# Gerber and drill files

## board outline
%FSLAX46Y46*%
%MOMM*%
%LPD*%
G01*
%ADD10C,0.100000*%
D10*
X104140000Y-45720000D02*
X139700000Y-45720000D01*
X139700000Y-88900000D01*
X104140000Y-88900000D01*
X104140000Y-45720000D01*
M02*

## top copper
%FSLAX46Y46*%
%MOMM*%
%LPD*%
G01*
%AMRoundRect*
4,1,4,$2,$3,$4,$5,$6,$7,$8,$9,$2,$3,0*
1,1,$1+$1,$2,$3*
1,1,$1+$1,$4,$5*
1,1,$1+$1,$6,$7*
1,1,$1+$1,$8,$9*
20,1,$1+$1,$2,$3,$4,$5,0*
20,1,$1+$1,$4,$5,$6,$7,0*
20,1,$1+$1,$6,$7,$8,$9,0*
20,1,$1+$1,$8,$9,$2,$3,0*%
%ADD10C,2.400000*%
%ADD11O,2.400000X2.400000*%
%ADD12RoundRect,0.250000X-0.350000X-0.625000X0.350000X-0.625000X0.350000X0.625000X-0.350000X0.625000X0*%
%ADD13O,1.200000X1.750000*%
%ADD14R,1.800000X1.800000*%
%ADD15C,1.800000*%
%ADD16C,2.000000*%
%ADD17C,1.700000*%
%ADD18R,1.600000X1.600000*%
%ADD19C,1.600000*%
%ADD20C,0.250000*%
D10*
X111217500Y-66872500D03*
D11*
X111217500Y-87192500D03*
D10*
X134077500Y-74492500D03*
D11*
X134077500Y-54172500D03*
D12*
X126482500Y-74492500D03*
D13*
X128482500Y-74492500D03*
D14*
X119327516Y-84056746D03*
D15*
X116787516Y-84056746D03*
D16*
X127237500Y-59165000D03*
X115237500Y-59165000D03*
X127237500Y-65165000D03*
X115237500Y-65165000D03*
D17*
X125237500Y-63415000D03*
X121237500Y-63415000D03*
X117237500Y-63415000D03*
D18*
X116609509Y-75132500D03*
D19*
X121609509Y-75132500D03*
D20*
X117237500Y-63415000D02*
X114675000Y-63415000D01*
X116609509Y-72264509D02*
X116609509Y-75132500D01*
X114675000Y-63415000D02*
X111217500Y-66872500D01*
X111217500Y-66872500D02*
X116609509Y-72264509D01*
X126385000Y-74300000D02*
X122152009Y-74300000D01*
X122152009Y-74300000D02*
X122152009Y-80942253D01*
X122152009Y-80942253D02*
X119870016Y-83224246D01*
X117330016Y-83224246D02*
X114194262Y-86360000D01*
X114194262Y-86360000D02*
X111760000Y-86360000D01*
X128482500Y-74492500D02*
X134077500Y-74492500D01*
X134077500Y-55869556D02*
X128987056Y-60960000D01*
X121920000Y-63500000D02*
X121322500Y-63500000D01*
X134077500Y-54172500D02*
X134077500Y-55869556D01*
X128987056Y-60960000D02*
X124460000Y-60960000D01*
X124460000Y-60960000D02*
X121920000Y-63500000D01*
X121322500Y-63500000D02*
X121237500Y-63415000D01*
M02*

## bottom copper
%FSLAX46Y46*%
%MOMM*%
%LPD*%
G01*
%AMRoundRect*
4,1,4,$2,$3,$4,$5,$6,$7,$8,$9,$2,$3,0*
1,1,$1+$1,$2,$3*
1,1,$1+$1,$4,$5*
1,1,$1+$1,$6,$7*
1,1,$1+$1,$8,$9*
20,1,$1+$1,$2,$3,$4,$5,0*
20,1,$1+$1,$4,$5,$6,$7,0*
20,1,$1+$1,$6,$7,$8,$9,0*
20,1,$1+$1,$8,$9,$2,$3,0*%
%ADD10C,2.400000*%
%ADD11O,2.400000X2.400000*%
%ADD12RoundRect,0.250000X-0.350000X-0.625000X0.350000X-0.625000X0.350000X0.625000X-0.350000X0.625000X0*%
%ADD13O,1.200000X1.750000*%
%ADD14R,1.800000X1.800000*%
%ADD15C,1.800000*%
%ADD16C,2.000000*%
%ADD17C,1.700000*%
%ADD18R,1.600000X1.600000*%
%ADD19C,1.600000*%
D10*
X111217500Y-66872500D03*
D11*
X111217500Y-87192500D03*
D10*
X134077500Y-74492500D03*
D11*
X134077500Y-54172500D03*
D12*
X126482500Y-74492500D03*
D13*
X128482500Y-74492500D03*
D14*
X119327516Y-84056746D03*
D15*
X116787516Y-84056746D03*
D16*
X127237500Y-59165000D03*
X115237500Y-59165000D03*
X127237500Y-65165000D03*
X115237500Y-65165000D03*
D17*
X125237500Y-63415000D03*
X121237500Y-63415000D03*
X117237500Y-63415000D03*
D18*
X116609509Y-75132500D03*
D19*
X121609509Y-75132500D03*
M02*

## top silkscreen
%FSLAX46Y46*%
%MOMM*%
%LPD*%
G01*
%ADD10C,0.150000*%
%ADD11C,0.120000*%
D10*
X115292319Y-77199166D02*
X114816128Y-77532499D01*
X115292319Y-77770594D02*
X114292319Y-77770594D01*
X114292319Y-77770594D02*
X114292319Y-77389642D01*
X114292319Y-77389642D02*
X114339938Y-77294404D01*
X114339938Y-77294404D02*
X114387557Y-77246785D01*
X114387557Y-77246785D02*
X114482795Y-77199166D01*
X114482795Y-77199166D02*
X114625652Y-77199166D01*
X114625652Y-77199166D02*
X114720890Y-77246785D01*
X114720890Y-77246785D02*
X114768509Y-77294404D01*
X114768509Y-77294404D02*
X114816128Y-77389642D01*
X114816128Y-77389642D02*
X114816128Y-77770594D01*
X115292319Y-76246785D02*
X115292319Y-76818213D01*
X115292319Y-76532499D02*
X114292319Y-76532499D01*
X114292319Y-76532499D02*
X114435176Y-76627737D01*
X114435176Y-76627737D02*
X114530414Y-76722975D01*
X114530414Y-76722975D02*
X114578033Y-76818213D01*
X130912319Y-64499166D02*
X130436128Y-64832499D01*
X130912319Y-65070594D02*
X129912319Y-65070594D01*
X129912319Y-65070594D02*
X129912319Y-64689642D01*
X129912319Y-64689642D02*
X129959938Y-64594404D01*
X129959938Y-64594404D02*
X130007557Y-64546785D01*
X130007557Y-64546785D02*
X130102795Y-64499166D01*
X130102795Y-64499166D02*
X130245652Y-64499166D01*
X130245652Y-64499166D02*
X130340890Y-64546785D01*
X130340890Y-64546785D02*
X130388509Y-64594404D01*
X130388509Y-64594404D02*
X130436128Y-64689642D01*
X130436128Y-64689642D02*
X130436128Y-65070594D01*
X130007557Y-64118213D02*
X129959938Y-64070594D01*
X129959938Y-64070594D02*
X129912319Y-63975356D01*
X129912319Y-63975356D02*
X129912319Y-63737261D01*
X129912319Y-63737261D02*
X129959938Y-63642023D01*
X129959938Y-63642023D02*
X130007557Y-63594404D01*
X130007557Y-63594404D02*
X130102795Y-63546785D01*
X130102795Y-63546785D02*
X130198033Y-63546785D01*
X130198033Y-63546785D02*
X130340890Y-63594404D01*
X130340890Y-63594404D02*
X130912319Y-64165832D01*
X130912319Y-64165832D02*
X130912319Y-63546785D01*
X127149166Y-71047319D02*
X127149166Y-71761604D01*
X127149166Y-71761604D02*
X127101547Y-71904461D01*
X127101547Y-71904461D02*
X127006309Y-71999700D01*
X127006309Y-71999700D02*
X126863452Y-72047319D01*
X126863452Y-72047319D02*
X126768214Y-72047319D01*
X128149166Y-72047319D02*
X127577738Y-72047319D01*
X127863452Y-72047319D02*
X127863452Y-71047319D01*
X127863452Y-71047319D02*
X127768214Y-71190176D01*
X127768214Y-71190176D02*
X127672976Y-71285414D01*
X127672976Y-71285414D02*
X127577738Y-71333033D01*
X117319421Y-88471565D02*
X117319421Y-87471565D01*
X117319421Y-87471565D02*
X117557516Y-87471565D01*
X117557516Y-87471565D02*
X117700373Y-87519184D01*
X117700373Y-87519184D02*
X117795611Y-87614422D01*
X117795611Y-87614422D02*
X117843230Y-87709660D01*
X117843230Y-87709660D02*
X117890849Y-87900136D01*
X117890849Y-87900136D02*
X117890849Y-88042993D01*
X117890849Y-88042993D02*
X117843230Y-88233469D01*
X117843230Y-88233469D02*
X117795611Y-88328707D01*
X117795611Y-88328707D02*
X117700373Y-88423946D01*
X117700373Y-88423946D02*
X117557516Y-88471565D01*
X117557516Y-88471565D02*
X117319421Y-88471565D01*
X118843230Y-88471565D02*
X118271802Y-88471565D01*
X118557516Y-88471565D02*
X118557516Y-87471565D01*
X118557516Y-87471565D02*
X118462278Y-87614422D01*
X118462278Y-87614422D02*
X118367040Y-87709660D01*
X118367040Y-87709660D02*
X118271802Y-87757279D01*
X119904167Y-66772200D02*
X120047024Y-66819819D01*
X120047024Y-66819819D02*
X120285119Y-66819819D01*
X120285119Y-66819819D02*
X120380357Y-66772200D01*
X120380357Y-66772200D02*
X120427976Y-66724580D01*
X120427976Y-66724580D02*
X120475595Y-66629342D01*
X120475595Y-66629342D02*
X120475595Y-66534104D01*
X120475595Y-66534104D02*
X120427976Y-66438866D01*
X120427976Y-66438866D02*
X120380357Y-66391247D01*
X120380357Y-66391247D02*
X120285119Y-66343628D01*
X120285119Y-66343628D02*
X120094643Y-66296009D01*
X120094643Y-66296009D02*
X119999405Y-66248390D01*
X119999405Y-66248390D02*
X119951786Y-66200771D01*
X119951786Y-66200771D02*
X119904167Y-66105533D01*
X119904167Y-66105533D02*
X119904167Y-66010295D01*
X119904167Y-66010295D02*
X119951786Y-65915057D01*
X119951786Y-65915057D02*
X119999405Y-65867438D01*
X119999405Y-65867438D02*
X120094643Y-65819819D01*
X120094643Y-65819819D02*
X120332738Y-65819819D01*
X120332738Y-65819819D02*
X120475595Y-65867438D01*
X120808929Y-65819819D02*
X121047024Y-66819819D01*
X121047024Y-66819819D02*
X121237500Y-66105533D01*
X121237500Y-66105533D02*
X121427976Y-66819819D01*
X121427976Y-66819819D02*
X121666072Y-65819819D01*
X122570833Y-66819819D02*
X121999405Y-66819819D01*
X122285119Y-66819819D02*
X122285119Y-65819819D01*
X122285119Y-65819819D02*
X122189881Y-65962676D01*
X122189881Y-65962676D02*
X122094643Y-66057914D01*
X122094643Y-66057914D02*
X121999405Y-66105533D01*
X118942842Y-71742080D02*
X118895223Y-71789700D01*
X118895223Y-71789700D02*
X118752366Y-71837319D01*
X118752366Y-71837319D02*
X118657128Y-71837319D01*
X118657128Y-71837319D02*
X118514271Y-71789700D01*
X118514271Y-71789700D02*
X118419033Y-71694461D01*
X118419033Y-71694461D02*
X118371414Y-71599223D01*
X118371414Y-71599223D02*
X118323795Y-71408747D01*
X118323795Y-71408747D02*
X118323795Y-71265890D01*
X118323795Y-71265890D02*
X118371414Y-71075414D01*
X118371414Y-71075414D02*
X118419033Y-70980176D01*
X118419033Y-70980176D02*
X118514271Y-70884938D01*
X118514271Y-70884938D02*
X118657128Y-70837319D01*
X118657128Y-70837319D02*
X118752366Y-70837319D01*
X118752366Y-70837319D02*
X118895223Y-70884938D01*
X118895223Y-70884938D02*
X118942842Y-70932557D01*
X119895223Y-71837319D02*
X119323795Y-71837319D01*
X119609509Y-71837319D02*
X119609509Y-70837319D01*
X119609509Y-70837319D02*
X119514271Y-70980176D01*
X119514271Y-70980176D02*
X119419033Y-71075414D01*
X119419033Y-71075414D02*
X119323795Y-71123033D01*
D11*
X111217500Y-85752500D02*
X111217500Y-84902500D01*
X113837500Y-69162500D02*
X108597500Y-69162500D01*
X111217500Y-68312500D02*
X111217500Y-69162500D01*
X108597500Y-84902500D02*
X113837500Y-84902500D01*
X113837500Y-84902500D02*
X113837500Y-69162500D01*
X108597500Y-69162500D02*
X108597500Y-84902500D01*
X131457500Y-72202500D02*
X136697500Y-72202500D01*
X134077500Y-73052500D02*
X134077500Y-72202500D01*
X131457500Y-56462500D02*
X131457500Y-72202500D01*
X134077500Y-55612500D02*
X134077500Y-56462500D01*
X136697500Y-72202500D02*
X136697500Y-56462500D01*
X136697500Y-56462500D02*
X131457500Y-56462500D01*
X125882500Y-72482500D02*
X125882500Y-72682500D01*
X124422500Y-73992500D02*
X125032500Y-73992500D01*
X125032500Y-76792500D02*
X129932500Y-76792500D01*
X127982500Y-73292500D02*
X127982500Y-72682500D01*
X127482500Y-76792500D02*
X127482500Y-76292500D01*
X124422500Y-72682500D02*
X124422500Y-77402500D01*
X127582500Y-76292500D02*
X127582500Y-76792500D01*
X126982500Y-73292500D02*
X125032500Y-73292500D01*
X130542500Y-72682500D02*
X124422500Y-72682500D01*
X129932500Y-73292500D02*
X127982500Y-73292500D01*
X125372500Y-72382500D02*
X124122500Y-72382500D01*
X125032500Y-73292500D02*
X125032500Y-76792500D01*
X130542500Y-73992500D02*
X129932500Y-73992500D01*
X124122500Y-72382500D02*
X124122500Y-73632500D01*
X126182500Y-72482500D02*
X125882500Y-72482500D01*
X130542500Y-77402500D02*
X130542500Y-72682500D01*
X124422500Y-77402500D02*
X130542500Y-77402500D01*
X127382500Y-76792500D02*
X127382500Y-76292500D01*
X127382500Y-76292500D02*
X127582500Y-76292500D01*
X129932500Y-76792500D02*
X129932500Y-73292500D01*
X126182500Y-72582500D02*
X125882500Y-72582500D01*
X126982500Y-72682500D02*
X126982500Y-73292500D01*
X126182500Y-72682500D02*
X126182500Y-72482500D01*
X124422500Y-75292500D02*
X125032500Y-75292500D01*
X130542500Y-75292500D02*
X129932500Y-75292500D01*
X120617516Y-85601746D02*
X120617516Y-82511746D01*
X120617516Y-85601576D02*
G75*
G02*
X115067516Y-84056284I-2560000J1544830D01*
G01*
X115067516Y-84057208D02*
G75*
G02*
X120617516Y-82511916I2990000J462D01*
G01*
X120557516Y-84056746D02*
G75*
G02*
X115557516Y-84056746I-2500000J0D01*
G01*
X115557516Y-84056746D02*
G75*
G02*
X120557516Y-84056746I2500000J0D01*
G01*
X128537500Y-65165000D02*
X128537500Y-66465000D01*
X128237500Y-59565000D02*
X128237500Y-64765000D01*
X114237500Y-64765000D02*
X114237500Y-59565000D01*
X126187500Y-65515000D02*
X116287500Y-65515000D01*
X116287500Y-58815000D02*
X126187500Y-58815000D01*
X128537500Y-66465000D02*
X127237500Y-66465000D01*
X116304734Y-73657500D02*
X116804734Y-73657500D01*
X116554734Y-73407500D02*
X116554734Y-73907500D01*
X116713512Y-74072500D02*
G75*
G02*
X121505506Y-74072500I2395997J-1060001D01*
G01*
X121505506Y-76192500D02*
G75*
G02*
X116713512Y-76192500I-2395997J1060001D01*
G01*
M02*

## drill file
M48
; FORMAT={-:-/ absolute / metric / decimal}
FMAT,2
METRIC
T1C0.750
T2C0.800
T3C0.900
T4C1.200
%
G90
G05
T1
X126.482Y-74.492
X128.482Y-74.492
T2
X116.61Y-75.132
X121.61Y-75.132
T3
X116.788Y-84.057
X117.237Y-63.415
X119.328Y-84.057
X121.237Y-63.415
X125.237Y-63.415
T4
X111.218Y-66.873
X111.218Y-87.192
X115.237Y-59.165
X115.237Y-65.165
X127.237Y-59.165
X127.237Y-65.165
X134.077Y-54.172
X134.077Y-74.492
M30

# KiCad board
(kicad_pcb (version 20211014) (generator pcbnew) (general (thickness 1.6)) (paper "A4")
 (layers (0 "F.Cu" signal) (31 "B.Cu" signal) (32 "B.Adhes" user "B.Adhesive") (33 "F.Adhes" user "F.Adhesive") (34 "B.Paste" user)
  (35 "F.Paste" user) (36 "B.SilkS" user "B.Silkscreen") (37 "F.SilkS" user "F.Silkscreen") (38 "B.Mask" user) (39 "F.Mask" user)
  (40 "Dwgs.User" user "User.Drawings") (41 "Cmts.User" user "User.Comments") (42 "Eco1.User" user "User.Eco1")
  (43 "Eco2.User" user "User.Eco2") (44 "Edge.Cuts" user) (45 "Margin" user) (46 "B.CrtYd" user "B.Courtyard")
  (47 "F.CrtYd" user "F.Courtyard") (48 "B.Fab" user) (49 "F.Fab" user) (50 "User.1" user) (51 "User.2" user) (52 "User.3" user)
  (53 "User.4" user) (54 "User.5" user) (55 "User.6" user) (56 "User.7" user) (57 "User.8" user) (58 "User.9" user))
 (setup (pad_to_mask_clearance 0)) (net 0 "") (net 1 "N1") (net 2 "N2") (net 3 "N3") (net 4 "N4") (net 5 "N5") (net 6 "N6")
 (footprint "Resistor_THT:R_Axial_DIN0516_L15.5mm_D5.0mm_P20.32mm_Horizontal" (layer "F.Cu") (at 111.2175 66.8725 -90)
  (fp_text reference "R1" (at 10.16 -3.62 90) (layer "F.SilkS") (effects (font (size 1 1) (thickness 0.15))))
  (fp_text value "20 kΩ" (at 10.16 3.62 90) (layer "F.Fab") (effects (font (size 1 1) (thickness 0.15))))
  (fp_line (start 18.88 0) (end 18.03 0) (layer "F.SilkS") (width 0.12))
  (fp_line (start 2.29 -2.62) (end 2.29 2.62) (layer "F.SilkS") (width 0.12))
  (fp_line (start 1.44 0) (end 2.29 0) (layer "F.SilkS") (width 0.12))
  (fp_line (start 18.03 2.62) (end 18.03 -2.62) (layer "F.SilkS") (width 0.12))
  (fp_line (start 18.03 -2.62) (end 2.29 -2.62) (layer "F.SilkS") (width 0.12))
  (fp_line (start 2.29 2.62) (end 18.03 2.62) (layer "F.SilkS") (width 0.12))
  (pad "1" thru_hole circle (at 0 0 270) (size 2.4 2.4) (drill 1.2) (layers *.Cu *.Mask) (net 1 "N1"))
  (pad "2" thru_hole oval (at 20.32 0 270) (size 2.4 2.4) (drill 1.2) (layers *.Cu *.Mask) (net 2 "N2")))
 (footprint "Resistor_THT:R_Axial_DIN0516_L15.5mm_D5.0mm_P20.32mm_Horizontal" (layer "F.Cu") (at 134.0775 74.4925 90)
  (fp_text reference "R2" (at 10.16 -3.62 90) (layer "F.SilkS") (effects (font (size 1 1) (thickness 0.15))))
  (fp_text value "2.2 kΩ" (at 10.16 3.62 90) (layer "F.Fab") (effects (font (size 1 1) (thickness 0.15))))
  (fp_line (start 2.29 -2.62) (end 2.29 2.62) (layer "F.SilkS") (width 0.12))
  (fp_line (start 1.44 0) (end 2.29 0) (layer "F.SilkS") (width 0.12))
  (fp_line (start 18.03 -2.62) (end 2.29 -2.62) (layer "F.SilkS") (width 0.12))
  (fp_line (start 18.88 0) (end 18.03 0) (layer "F.SilkS") (width 0.12))
  (fp_line (start 2.29 2.62) (end 18.03 2.62) (layer "F.SilkS") (width 0.12))
  (fp_line (start 18.03 2.62) (end 18.03 -2.62) (layer "F.SilkS") (width 0.12))
  (pad "1" thru_hole circle (at 0 0 90) (size 2.4 2.4) (drill 1.2) (layers *.Cu *.Mask) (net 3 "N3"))
  (pad "2" thru_hole oval (at 20.32 0 90) (size 2.4 2.4) (drill 1.2) (layers *.Cu *.Mask) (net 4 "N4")))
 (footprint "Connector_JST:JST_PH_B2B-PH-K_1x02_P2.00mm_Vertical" (layer "F.Cu") (at 126.4825 74.4925)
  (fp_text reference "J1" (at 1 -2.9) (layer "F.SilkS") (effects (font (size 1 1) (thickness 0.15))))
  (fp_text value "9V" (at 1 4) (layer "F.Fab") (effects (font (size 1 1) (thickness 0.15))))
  (fp_line (start -0.6 -2.01) (end -0.6 -1.81) (layer "F.SilkS") (width 0.12))
  (fp_line (start -2.06 -0.5) (end -1.45 -0.5) (layer "F.SilkS") (width 0.12))
  (fp_line (start -1.45 2.3) (end 3.45 2.3) (layer "F.SilkS") (width 0.12))
  (fp_line (start 1.5 -1.2) (end 1.5 -1.81) (layer "F.SilkS") (width 0.12))
  (fp_line (start 1 2.3) (end 1 1.8) (layer "F.SilkS") (width 0.12))
  (fp_line (start -2.06 -1.81) (end -2.06 2.91) (layer "F.SilkS") (width 0.12))
  (fp_line (start 1.1 1.8) (end 1.1 2.3) (layer "F.SilkS") (width 0.12))
  (fp_line (start 0.5 -1.2) (end -1.45 -1.2) (layer "F.SilkS") (width 0.12))
  (fp_line (start 4.06 -1.81) (end -2.06 -1.81) (layer "F.SilkS") (width 0.12))
  (fp_line (start 3.45 -1.2) (end 1.5 -1.2) (layer "F.SilkS") (width 0.12))
  (fp_line (start -1.11 -2.11) (end -2.36 -2.11) (layer "F.SilkS") (width 0.12))
  (fp_line (start -1.45 -1.2) (end -1.45 2.3) (layer "F.SilkS") (width 0.12))
  (fp_line (start 4.06 -0.5) (end 3.45 -0.5) (layer "F.SilkS") (width 0.12))
  (fp_line (start -2.36 -2.11) (end -2.36 -0.86) (layer "F.SilkS") (width 0.12))
  (fp_line (start -0.3 -2.01) (end -0.6 -2.01) (layer "F.SilkS") (width 0.12))
  (fp_line (start 4.06 2.91) (end 4.06 -1.81) (layer "F.SilkS") (width 0.12))
  (fp_line (start -2.06 2.91) (end 4.06 2.91) (layer "F.SilkS") (width 0.12))
  (fp_line (start 0.9 2.3) (end 0.9 1.8) (layer "F.SilkS") (width 0.12))
  (fp_line (start 0.9 1.8) (end 1.1 1.8) (layer "F.SilkS") (width 0.12))
  (fp_line (start 3.45 2.3) (end 3.45 -1.2) (layer "F.SilkS") (width 0.12))
  (fp_line (start -0.3 -1.91) (end -0.6 -1.91) (layer "F.SilkS") (width 0.12))
  (fp_line (start 0.5 -1.81) (end 0.5 -1.2) (layer "F.SilkS") (width 0.12))
  (fp_line (start -0.3 -1.81) (end -0.3 -2.01) (layer "F.SilkS") (width 0.12))
  (fp_line (start -2.06 0.8) (end -1.45 0.8) (layer "F.SilkS") (width 0.12))
  (fp_line (start 4.06 0.8) (end 3.45 0.8) (layer "F.SilkS") (width 0.12))
  (pad "1" thru_hole roundrect (at 0 0) (size 1.2 1.75) (drill 0.75) (layers *.Cu *.Mask) (roundrect_rratio 0.2083333333) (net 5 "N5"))
  (pad "2" thru_hole oval (at 2 0) (size 1.2 1.75) (drill 0.75) (layers *.Cu *.Mask) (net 3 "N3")))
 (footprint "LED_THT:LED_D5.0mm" (layer "F.Cu") (at 119.327516 84.056746 180)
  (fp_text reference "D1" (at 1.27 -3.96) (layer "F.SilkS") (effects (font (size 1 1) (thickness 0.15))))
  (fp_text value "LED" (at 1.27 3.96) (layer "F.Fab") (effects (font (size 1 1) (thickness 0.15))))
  (fp_line (start -1.29 -1.545) (end -1.29 1.545) (layer "F.SilkS") (width 0.12))
  (fp_arc (start -1.29 -1.54483) (mid 2.072002 -2.880433) (end 4.26 0.000462) (layer "F.SilkS") (width 0.12))
  (fp_arc (start 4.26 -0.000462) (mid 2.072002 2.880433) (end -1.29 1.54483) (layer "F.SilkS") (width 0.12))
  (fp_circle (center 1.27 0) (end 3.77 0) (layer "F.SilkS") (width 0.12) (fill none))
  (pad "1" thru_hole rect (at 0 0 180) (size 1.8 1.8) (drill 0.9) (layers *.Cu *.Mask) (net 5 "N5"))
  (pad "2" thru_hole circle (at 2.54 0 180) (size 1.8 1.8) (drill 0.9) (layers *.Cu *.Mask) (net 2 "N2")))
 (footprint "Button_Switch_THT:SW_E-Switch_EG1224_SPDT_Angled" (layer "F.Cu") (at 125.2375 63.415 180)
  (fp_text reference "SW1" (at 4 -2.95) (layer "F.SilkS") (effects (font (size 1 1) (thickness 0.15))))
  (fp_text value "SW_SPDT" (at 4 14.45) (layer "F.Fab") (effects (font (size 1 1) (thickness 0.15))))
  (fp_line (start -3.3 -1.75) (end -3.3 -3.05) (layer "F.SilkS") (width 0.12))
  (fp_line (start -3 3.85) (end -3 -1.35) (layer "F.SilkS") (width 0.12))
  (fp_line (start 11 -1.35) (end 11 3.85) (layer "F.SilkS") (width 0.12))
  (fp_line (start -0.95 -2.1) (end 8.95 -2.1) (layer "F.SilkS") (width 0.12))
  (fp_line (start 8.95 4.6) (end -0.95 4.6) (layer "F.SilkS") (width 0.12))
  (fp_line (start -3.3 -3.05) (end -2 -3.05) (layer "F.SilkS") (width 0.12))
  (pad "" thru_hole circle (at -2 4.25 180) (size 2 2) (drill 1.2) (layers *.Cu *.Mask))
  (pad "" thru_hole circle (at 10 4.25 180) (size 2 2) (drill 1.2) (layers *.Cu *.Mask))
  (pad "" thru_hole circle (at -2 -1.75 180) (size 2 2) (drill 1.2) (layers *.Cu *.Mask))
  (pad "" thru_hole circle (at 10 -1.75 180) (size 2 2) (drill 1.2) (layers *.Cu *.Mask))
  (pad "1" thru_hole circle (at 0 0 180) (size 1.7 1.7) (drill 0.9) (layers *.Cu *.Mask) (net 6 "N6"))
  (pad "2" thru_hole circle (at 4 0 180) (size 1.7 1.7) (drill 0.9) (layers *.Cu *.Mask) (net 4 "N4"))
  (pad "3" thru_hole circle (at 8 0 180) (size 1.7 1.7) (drill 0.9) (layers *.Cu *.Mask) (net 1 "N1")))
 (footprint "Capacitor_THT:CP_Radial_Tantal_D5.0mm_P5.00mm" (layer "F.Cu") (at 116.609509 75.1325)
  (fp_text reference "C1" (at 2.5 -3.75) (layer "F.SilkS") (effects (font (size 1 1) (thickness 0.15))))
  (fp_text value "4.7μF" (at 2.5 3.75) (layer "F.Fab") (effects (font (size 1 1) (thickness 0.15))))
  (fp_line (start -0.304775 -1.475) (end 0.195225 -1.475) (layer "F.SilkS") (width 0.12))
  (fp_line (start -0.054775 -1.725) (end -0.054775 -1.225) (layer "F.SilkS") (width 0.12))
  (fp_arc (start 0.104003 -1.06) (mid 2.5 -2.62) (end 4.895997 -1.06) (layer "F.SilkS") (width 0.12))
  (fp_arc (start 4.895997 1.06) (mid 2.5 2.62) (end 0.104003 1.06) (layer "F.SilkS") (width 0.12))
  (pad "1" thru_hole rect (at 0 0) (size 1.6 1.6) (drill 0.8) (layers *.Cu *.Mask) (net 1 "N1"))
  (pad "2" thru_hole circle (at 5 0) (size 1.6 1.6) (drill 0.8) (layers *.Cu *.Mask) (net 5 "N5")))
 (gr_rect (start 104.14 45.72) (end 139.7 88.9) (layer "Edge.Cuts") (width 0.1) (fill none))
 (segment (start 117.2375 63.415) (end 114.675 63.415) (width 0.25) (layer "F.Cu") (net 1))
 (segment (start 116.609509 72.264509) (end 116.609509 75.1325) (width 0.25) (layer "F.Cu") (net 1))
 (segment (start 114.675 63.415) (end 111.2175 66.8725) (width 0.25) (layer "F.Cu") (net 1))
 (segment (start 111.2175 66.8725) (end 116.609509 72.264509) (width 0.25) (layer "F.Cu") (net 1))
 (segment (start 126.385 74.3) (end 122.152009 74.3) (width 0.25) (layer "F.Cu") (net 5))
 (segment (start 122.152009 74.3) (end 122.152009 80.942253) (width 0.25) (layer "F.Cu") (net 5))
 (segment (start 122.152009 80.942253) (end 119.870016 83.224246) (width 0.25) (layer "F.Cu") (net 5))
 (segment (start 117.330016 83.224246) (end 114.194262 86.36) (width 0.25) (layer "F.Cu") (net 2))
 (segment (start 114.194262 86.36) (end 111.76 86.36) (width 0.25) (layer "F.Cu") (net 2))
 (segment (start 128.4825 74.4925) (end 134.0775 74.4925) (width 0.25) (layer "F.Cu") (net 3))
 (segment (start 134.0775 55.869556) (end 128.987056 60.96) (width 0.25) (layer "F.Cu") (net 4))
 (segment (start 121.92 63.5) (end 121.3225 63.5) (width 0.25) (layer "F.Cu") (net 4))
 (segment (start 134.0775 54.1725) (end 134.0775 55.869556) (width 0.25) (layer "F.Cu") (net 4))
 (segment (start 128.987056 60.96) (end 124.46 60.96) (width 0.25) (layer "F.Cu") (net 4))
 (segment (start 124.46 60.96) (end 121.92 63.5) (width 0.25) (layer "F.Cu") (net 4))
 (segment (start 121.3225 63.5) (end 121.2375 63.415) (width 0.25) (layer "F.Cu") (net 4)))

